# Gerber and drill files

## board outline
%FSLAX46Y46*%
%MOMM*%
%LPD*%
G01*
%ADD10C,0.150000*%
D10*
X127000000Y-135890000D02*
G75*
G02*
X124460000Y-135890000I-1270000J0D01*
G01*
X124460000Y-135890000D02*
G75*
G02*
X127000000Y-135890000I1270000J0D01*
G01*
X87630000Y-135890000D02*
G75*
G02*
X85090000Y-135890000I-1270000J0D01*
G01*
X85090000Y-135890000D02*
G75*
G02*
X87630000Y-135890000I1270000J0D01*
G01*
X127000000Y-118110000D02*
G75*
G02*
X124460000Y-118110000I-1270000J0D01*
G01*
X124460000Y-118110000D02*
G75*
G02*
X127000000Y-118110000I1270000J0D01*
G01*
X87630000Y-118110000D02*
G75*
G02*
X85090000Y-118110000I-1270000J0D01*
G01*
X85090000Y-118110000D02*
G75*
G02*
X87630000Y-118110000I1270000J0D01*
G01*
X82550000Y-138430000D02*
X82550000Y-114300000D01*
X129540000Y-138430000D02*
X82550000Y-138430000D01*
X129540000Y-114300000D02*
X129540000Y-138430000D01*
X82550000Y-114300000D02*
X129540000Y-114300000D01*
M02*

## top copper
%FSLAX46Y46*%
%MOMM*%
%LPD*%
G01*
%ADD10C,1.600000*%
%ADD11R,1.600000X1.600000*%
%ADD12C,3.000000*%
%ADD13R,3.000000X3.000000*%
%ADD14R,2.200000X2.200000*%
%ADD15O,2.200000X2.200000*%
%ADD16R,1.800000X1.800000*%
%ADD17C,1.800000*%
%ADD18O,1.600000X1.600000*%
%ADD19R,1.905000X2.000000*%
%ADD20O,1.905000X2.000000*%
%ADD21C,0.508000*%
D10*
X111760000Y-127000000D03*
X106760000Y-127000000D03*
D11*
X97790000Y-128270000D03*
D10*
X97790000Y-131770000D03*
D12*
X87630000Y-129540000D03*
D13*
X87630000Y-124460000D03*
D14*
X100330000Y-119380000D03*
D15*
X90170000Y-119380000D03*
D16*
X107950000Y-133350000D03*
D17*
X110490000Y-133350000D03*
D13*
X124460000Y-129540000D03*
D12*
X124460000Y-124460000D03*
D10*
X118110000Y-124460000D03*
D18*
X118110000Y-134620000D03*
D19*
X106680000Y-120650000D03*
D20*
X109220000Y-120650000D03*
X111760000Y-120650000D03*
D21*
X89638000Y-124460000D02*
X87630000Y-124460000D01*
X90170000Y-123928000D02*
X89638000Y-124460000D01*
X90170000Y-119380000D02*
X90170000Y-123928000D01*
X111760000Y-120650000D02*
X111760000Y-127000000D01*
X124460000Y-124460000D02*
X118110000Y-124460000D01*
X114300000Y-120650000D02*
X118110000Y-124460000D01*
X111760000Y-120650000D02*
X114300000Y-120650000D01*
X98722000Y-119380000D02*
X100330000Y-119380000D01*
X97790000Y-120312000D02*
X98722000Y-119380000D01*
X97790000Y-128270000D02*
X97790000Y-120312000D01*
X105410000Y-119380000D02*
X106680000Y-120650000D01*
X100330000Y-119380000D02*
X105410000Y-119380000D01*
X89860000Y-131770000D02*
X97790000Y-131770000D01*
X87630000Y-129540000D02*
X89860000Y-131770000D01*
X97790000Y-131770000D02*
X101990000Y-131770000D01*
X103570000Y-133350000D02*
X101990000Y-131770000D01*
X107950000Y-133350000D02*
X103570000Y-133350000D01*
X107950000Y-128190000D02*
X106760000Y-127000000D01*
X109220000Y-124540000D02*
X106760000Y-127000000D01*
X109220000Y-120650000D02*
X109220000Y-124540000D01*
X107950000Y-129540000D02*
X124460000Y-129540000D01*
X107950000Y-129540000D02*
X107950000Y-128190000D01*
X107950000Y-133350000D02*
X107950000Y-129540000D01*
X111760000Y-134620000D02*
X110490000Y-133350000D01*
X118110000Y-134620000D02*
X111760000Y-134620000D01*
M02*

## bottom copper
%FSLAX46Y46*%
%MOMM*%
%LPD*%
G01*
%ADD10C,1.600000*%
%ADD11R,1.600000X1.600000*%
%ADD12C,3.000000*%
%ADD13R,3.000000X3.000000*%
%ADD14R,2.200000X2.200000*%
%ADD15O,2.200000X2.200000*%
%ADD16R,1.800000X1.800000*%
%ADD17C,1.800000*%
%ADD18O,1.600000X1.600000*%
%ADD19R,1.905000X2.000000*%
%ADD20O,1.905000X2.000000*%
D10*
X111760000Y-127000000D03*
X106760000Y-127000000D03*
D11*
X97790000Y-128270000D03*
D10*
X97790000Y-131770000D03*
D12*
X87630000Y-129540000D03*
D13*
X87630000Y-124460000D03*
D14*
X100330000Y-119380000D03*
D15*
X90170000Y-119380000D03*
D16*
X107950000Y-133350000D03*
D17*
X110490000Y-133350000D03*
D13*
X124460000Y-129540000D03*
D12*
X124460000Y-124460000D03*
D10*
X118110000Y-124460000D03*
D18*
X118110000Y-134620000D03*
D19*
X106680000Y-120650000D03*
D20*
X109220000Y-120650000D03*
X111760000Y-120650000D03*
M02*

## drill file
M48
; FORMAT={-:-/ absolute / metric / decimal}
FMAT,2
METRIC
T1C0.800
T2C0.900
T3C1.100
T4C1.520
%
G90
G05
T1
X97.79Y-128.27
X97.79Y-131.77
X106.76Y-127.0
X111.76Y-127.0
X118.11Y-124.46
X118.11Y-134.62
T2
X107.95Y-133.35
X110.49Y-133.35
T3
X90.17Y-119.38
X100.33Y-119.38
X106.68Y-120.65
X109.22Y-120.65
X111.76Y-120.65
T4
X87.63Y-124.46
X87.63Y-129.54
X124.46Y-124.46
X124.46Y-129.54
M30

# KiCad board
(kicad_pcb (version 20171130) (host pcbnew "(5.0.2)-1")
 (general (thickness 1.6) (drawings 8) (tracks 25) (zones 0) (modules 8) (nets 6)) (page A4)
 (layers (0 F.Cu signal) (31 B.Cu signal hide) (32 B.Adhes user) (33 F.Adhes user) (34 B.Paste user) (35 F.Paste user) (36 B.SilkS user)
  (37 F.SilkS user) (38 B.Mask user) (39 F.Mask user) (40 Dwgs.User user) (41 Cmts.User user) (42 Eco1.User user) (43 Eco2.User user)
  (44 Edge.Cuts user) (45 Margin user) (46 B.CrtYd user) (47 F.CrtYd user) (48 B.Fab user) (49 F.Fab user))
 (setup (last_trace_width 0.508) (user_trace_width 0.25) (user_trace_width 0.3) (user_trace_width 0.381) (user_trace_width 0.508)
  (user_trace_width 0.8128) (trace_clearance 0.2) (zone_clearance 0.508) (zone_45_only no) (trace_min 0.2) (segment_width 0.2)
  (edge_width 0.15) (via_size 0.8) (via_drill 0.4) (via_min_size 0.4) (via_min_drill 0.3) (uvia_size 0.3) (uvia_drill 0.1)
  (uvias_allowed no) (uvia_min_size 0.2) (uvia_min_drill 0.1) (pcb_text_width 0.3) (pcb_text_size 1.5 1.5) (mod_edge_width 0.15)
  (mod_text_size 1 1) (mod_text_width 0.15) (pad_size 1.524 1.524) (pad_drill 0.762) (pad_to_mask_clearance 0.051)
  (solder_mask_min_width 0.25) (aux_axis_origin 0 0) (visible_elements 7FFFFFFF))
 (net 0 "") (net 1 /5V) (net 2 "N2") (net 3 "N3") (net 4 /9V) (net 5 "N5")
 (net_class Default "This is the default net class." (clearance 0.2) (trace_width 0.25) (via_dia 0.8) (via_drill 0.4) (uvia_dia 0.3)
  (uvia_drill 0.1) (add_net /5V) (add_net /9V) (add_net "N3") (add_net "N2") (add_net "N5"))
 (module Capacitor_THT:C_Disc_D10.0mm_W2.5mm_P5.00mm (layer F.Cu) (at 111.76 127 180)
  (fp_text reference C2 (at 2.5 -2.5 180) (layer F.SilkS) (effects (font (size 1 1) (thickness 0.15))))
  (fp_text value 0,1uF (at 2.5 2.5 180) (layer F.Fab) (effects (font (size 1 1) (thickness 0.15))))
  (pad 1 thru_hole circle (at 0 0 180) (size 1.6 1.6) (drill 0.8) (layers *.Cu *.Mask) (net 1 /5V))
  (pad 2 thru_hole circle (at 5 0 180) (size 1.6 1.6) (drill 0.8) (layers *.Cu *.Mask) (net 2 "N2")))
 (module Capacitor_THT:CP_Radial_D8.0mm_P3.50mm (layer F.Cu) (at 97.79 128.27 270)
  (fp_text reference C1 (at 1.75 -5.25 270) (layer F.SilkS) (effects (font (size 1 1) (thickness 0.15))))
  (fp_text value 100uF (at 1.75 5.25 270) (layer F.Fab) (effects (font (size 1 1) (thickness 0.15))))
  (pad 1 thru_hole rect (at 0 0 270) (size 1.6 1.6) (drill 0.8) (layers *.Cu *.Mask) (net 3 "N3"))
  (pad 2 thru_hole circle (at 3.5 0 270) (size 1.6 1.6) (drill 0.8) (layers *.Cu *.Mask) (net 2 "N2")))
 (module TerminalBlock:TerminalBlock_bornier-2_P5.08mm (layer F.Cu) (at 87.63 124.46 270)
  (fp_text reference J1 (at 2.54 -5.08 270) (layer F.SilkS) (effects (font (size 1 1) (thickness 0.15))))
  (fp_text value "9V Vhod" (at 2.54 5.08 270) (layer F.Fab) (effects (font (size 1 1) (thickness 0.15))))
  (pad 2 thru_hole circle (at 5.08 0 270) (size 3 3) (drill 1.52) (layers *.Cu *.Mask) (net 2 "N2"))
  (pad 1 thru_hole rect (at 0 0 270) (size 3 3) (drill 1.52) (layers *.Cu *.Mask) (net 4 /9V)))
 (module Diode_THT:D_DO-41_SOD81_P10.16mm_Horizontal (layer F.Cu) (at 100.33 119.38 180)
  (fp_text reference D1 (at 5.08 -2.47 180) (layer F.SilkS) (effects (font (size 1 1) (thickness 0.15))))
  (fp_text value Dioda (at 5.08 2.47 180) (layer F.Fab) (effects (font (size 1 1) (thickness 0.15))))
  (pad 1 thru_hole rect (at 0 0 180) (size 2.2 2.2) (drill 1.1) (layers *.Cu *.Mask) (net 3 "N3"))
  (pad 2 thru_hole oval (at 10.16 0 180) (size 2.2 2.2) (drill 1.1) (layers *.Cu *.Mask) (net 4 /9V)))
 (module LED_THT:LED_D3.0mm (layer F.Cu) (at 107.95 133.35)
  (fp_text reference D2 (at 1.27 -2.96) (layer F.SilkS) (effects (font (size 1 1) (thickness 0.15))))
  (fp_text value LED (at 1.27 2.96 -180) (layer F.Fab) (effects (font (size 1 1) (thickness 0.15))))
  (pad 1 thru_hole rect (at 0 0) (size 1.8 1.8) (drill 0.9) (layers *.Cu *.Mask) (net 2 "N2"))
  (pad 2 thru_hole circle (at 2.54 0) (size 1.8 1.8) (drill 0.9) (layers *.Cu *.Mask) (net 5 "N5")))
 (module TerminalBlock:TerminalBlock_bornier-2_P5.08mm (layer F.Cu) (at 124.46 129.54 90)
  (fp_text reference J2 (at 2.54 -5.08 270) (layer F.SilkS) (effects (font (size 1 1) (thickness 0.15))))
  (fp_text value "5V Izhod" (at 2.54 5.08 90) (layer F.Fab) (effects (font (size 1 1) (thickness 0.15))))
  (pad 1 thru_hole rect (at 0 0 90) (size 3 3) (drill 1.52) (layers *.Cu *.Mask) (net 2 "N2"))
  (pad 2 thru_hole circle (at 5.08 0 90) (size 3 3) (drill 1.52) (layers *.Cu *.Mask) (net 1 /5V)))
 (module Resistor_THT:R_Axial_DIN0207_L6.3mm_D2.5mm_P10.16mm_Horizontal (layer F.Cu) (at 118.11 124.46 270)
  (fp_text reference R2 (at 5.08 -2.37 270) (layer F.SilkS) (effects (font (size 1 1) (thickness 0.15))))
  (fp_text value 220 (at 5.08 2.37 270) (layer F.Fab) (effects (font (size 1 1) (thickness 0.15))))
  (pad 1 thru_hole circle (at 0 0 270) (size 1.6 1.6) (drill 0.8) (layers *.Cu *.Mask) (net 1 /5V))
  (pad 2 thru_hole oval (at 10.16 0 270) (size 1.6 1.6) (drill 0.8) (layers *.Cu *.Mask) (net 5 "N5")))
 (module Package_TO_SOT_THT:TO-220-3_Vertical (layer F.Cu) (at 106.68 120.65)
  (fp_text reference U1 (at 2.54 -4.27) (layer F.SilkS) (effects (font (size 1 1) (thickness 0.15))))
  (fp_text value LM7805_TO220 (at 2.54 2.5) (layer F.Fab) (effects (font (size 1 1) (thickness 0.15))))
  (pad 1 thru_hole rect (at 0 0) (size 1.905 2) (drill 1.1) (layers *.Cu *.Mask) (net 3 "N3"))
  (pad 2 thru_hole oval (at 2.54 0) (size 1.905 2) (drill 1.1) (layers *.Cu *.Mask) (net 2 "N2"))
  (pad 3 thru_hole oval (at 5.08 0) (size 1.905 2) (drill 1.1) (layers *.Cu *.Mask) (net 1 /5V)))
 (gr_circle (center 125.73 135.89) (end 125.73 134.62) (layer Edge.Cuts) (width 0.15))
 (gr_circle (center 86.36 135.89) (end 87.63 135.89) (layer Edge.Cuts) (width 0.15))
 (gr_circle (center 125.73 118.11) (end 127 118.11) (layer Edge.Cuts) (width 0.15))
 (gr_circle (center 86.36 118.11) (end 86.36 116.84) (layer Edge.Cuts) (width 0.15))
 (gr_line (start 82.55 138.43) (end 82.55 114.3) (layer Edge.Cuts) (width 0.15))
 (gr_line (start 129.54 138.43) (end 82.55 138.43) (layer Edge.Cuts) (width 0.15))
 (gr_line (start 129.54 114.3) (end 129.54 138.43) (layer Edge.Cuts) (width 0.15))
 (gr_line (start 82.55 114.3) (end 129.54 114.3) (layer Edge.Cuts) (width 0.15))
 (segment (start 89.638 124.46) (end 87.63 124.46) (width 0.508) (layer F.Cu) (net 4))
 (segment (start 90.17 123.928) (end 89.638 124.46) (width 0.508) (layer F.Cu) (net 4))
 (segment (start 90.17 119.38) (end 90.17 123.928) (width 0.508) (layer F.Cu) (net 4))
 (segment (start 111.76 120.65) (end 111.76 127) (width 0.508) (layer F.Cu) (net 1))
 (segment (start 124.46 124.46) (end 118.11 124.46) (width 0.508) (layer F.Cu) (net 1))
 (segment (start 114.3 120.65) (end 118.11 124.46) (width 0.508) (layer F.Cu) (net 1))
 (segment (start 111.76 120.65) (end 114.3 120.65) (width 0.508) (layer F.Cu) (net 1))
 (segment (start 98.722 119.38) (end 100.33 119.38) (width 0.508) (layer F.Cu) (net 3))
 (segment (start 97.79 120.312) (end 98.722 119.38) (width 0.508) (layer F.Cu) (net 3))
 (segment (start 97.79 128.27) (end 97.79 120.312) (width 0.508) (layer F.Cu) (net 3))
 (segment (start 105.41 119.38) (end 106.68 120.65) (width 0.508) (layer F.Cu) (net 3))
 (segment (start 100.33 119.38) (end 105.41 119.38) (width 0.508) (layer F.Cu) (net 3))
 (segment (start 89.86 131.77) (end 97.79 131.77) (width 0.508) (layer F.Cu) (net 2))
 (segment (start 87.63 129.54) (end 89.86 131.77) (width 0.508) (layer F.Cu) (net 2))
 (segment (start 97.79 131.77) (end 101.99 131.77) (width 0.508) (layer F.Cu) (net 2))
 (segment (start 103.57 133.35) (end 101.99 131.77) (width 0.508) (layer F.Cu) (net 2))
 (segment (start 107.95 133.35) (end 103.57 133.35) (width 0.508) (layer F.Cu) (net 2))
 (segment (start 107.95 128.19) (end 106.76 127) (width 0.508) (layer F.Cu) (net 2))
 (segment (start 109.22 124.54) (end 106.76 127) (width 0.508) (layer F.Cu) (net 2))
 (segment (start 109.22 120.65) (end 109.22 124.54) (width 0.508) (layer F.Cu) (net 2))
 (segment (start 107.95 129.54) (end 124.46 129.54) (width 0.508) (layer F.Cu) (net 2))
 (segment (start 107.95 129.54) (end 107.95 128.19) (width 0.508) (layer F.Cu) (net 2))
 (segment (start 107.95 133.35) (end 107.95 129.54) (width 0.508) (layer F.Cu) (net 2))
 (segment (start 111.76 134.62) (end 110.49 133.35) (width 0.508) (layer F.Cu) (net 5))
 (segment (start 118.11 134.62) (end 111.76 134.62) (width 0.508) (layer F.Cu) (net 5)))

